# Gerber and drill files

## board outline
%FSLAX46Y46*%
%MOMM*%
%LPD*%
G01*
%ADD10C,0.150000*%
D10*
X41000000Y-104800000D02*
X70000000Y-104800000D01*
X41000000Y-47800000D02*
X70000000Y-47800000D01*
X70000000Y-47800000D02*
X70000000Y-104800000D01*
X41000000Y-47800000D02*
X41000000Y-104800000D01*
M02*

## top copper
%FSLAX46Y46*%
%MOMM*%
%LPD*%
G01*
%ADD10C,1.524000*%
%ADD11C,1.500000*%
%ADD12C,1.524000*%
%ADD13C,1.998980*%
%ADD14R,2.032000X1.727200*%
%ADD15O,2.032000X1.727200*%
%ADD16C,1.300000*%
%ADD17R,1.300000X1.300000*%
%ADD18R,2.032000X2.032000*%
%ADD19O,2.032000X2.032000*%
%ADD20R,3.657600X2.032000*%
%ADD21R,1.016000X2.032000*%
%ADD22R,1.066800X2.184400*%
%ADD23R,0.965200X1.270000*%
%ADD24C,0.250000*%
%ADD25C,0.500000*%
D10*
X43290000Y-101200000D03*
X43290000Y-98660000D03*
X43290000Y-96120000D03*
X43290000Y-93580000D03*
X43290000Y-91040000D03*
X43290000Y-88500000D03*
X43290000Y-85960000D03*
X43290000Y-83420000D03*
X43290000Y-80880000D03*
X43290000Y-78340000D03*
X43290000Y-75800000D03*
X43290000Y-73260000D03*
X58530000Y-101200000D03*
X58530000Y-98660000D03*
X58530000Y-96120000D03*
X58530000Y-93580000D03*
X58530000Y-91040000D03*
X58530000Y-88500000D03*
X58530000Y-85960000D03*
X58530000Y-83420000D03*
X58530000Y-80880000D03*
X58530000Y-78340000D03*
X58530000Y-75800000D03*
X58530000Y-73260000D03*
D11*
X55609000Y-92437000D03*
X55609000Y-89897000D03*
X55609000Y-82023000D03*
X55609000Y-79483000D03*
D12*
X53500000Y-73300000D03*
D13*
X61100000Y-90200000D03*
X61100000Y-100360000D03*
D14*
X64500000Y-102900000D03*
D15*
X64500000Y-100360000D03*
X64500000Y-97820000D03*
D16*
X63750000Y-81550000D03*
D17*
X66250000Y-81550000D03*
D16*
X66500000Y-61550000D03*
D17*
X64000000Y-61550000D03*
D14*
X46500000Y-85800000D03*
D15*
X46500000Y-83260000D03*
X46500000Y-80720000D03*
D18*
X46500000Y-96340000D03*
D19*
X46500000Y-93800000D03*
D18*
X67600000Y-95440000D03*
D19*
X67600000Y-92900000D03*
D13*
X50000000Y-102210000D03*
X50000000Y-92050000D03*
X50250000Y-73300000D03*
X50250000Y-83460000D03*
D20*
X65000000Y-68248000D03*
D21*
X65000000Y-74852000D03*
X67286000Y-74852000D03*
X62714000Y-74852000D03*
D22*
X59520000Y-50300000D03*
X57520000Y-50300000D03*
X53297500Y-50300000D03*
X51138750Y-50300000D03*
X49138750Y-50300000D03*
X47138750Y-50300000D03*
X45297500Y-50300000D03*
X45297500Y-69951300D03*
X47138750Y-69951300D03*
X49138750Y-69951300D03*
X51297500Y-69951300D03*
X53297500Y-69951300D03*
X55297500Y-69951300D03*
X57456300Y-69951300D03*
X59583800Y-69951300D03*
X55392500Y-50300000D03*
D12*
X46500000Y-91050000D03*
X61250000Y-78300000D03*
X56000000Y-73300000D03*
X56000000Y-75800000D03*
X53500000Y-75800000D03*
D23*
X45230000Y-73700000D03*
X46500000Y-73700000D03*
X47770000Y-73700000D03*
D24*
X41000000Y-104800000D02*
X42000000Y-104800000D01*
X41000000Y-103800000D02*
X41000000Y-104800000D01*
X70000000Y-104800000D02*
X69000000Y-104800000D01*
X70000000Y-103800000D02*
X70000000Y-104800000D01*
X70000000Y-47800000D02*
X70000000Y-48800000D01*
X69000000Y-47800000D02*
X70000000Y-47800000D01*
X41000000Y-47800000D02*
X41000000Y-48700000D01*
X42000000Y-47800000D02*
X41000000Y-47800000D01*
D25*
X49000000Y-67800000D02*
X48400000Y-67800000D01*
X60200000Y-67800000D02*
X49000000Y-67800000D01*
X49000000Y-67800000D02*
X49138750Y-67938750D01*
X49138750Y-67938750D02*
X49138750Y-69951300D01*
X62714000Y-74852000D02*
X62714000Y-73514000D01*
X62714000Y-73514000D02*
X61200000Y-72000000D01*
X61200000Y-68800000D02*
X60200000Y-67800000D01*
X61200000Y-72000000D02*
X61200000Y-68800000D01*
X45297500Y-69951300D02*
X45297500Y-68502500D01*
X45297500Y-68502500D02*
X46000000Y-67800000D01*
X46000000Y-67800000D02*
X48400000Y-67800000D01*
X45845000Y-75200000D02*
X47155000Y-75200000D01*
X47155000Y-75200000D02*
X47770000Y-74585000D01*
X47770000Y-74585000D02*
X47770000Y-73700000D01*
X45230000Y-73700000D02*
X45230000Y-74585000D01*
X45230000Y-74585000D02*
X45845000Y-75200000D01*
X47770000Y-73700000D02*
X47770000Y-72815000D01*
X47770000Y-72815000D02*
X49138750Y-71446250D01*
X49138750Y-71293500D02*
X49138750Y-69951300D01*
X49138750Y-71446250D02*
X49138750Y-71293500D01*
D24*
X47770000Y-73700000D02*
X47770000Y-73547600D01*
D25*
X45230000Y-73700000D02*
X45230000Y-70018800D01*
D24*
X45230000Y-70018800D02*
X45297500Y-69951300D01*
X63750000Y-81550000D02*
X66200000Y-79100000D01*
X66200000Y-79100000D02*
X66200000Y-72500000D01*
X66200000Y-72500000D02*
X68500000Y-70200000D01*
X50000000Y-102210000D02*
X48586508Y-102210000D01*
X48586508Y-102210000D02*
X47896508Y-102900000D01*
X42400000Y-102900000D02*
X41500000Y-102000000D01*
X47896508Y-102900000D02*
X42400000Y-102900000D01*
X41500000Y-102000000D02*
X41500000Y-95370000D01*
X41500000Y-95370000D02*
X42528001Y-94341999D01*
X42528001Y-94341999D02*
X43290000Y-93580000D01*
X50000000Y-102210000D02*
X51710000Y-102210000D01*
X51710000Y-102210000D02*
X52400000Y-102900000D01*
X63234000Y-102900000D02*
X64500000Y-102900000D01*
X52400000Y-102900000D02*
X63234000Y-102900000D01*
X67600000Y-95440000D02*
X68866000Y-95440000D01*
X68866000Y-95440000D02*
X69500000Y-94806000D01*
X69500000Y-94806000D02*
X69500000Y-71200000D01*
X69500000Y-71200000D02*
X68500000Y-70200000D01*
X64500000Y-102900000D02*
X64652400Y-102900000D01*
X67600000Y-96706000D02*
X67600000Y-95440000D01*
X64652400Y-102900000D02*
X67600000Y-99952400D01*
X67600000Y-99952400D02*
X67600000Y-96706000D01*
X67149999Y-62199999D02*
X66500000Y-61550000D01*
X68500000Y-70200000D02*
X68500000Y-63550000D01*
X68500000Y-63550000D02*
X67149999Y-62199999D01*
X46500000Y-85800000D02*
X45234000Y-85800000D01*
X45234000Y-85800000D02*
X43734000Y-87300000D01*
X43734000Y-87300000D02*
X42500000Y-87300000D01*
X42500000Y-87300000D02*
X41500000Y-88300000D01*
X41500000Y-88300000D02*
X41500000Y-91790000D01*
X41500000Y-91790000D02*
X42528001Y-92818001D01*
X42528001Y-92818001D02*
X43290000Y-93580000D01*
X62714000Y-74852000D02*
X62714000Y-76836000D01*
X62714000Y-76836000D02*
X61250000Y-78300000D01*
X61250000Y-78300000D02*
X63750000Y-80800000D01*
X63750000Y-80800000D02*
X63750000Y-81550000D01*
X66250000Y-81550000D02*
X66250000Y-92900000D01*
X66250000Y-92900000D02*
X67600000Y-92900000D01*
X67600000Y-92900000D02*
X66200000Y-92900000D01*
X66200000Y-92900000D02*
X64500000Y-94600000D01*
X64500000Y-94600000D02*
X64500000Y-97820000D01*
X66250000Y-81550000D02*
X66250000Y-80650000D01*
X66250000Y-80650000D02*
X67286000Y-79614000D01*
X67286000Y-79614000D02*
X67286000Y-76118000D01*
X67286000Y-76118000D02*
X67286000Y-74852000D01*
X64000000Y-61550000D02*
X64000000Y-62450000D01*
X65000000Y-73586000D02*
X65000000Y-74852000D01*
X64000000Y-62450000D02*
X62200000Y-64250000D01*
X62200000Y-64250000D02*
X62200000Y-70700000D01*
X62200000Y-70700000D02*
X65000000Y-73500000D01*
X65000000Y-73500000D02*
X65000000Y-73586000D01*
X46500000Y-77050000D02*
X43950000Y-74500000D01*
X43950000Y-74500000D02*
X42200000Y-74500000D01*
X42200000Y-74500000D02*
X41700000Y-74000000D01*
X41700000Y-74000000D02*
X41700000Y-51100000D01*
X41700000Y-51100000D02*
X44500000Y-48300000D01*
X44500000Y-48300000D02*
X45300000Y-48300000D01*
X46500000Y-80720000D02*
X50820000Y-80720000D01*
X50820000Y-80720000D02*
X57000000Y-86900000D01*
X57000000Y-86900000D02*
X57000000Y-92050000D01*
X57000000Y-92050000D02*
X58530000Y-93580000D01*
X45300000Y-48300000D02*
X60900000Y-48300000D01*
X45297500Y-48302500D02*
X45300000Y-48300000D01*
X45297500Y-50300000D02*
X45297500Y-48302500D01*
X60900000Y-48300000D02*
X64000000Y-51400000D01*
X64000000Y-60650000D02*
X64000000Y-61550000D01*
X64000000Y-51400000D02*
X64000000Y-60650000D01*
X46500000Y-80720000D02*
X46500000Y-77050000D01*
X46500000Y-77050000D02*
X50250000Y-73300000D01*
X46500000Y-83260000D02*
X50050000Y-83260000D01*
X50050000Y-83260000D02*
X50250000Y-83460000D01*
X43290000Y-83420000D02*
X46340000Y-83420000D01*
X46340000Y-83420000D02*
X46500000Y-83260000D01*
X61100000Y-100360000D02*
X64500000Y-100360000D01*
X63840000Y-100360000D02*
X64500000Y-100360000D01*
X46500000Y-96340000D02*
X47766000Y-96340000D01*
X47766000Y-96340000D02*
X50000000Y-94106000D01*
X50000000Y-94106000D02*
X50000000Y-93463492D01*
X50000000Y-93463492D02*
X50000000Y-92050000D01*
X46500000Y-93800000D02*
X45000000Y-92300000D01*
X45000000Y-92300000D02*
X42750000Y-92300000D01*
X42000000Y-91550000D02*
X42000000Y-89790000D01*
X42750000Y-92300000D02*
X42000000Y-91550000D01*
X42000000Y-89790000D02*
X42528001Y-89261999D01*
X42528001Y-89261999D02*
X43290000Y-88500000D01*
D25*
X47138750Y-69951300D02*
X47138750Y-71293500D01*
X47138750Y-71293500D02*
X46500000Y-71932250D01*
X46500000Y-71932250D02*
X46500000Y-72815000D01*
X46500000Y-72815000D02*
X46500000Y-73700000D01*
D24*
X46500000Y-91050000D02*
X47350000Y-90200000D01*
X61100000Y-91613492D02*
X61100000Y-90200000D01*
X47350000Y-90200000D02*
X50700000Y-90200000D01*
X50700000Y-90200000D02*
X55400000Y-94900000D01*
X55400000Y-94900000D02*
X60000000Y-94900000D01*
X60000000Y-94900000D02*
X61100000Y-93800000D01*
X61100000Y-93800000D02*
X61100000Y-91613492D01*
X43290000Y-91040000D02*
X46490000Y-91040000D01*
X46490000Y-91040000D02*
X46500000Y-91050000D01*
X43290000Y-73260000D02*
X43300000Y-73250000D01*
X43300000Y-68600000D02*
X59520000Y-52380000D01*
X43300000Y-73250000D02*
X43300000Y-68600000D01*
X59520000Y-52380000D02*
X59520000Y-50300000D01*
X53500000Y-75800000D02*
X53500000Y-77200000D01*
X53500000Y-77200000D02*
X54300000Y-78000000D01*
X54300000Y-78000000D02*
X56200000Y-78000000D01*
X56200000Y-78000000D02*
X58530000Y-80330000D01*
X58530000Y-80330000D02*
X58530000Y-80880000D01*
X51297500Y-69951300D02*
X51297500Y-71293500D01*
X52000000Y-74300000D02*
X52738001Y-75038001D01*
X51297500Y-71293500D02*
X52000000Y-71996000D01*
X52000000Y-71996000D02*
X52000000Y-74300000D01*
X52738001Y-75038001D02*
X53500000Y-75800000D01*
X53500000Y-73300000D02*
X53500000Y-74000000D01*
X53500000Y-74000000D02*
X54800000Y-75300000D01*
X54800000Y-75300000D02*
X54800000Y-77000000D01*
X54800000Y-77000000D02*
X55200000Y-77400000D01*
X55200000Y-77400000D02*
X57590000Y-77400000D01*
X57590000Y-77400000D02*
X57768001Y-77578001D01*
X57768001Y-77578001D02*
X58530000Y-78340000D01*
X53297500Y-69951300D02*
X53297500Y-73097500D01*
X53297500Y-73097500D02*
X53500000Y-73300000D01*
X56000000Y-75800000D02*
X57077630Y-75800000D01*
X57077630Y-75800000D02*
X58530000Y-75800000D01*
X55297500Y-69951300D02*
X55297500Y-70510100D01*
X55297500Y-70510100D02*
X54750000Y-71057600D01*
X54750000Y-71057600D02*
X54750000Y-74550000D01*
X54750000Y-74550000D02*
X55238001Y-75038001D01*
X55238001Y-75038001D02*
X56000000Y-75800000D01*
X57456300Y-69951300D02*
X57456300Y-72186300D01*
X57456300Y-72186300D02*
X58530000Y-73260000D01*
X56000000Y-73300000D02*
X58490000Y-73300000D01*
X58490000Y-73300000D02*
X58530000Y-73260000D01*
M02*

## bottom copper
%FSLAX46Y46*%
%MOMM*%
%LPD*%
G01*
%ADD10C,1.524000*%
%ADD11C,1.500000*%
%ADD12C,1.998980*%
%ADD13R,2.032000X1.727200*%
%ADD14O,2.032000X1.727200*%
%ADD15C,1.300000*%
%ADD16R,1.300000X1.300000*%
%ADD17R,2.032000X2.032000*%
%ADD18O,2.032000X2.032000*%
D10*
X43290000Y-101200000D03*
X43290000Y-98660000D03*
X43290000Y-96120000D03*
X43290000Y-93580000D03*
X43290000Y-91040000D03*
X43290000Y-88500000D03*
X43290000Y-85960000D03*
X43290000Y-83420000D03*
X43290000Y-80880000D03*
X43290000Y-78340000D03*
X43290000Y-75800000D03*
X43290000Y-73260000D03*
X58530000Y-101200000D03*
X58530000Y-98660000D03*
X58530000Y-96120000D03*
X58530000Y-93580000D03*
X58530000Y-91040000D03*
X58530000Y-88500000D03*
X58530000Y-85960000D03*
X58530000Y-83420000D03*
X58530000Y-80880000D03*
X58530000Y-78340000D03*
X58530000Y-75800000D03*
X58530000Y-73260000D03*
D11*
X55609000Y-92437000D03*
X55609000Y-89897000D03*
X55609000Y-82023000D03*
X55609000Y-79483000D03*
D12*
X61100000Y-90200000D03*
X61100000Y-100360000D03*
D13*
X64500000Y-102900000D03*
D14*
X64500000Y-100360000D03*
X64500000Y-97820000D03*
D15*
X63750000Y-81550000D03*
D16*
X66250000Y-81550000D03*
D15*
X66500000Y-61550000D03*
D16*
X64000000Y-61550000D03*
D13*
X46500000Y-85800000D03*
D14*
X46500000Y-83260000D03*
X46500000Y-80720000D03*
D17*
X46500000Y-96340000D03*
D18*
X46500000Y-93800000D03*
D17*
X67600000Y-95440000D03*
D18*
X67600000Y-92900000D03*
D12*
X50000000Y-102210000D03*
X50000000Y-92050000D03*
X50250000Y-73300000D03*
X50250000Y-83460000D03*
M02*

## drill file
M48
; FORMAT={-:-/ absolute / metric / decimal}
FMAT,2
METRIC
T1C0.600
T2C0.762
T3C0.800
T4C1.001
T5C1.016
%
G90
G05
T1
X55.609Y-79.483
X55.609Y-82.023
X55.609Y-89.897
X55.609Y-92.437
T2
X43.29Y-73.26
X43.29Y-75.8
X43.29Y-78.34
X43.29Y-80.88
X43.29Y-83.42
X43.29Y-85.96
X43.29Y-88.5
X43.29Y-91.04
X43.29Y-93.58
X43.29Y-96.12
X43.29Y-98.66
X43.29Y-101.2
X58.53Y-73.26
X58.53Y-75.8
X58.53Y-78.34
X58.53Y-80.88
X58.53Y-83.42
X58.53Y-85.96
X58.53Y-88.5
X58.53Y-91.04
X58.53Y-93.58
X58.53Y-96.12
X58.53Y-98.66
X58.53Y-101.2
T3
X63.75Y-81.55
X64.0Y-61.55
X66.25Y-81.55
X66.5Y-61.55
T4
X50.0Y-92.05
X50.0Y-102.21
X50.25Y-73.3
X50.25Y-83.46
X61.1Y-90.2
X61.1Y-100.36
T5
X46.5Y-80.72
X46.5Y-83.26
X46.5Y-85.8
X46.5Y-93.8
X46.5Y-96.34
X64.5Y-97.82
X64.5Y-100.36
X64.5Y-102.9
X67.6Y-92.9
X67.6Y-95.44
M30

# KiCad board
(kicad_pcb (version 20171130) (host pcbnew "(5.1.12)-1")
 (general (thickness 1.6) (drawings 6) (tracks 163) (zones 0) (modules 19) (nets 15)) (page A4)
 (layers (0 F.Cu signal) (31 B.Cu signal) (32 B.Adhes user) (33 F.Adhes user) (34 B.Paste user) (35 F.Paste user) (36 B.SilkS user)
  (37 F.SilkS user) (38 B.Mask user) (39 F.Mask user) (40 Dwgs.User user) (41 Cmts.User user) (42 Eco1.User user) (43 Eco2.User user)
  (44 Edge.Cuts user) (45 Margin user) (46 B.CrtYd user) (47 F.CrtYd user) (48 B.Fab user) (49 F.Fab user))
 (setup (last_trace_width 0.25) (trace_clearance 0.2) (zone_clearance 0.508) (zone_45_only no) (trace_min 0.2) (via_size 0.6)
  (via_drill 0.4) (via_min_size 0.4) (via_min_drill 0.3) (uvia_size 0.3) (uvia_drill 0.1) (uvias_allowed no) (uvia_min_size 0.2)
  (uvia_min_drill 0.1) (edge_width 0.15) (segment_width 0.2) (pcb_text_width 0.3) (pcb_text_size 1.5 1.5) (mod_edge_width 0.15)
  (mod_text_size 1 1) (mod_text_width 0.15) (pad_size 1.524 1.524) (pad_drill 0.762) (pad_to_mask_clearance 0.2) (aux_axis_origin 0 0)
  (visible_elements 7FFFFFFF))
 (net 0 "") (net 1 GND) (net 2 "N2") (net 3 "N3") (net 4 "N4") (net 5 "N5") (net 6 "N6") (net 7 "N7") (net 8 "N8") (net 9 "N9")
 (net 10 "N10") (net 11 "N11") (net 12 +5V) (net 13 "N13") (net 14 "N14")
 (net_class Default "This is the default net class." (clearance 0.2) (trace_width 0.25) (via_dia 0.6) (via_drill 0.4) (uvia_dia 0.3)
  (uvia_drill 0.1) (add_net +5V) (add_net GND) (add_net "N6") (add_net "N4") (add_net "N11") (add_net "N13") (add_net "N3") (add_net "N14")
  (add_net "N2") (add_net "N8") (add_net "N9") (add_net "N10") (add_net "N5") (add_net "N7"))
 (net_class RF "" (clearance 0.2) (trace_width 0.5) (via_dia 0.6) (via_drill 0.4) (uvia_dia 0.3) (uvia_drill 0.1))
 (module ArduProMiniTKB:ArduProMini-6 (layer B.Cu) (at 40.75 107.55)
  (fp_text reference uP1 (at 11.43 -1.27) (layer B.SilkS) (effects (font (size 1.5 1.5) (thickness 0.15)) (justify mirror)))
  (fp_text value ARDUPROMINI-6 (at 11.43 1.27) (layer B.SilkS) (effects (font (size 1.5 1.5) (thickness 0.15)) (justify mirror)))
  (pad 7 thru_hole circle (at 2.54 -6.35) (size 1.524 1.524) (drill 0.762) (layers *.Cu *.Mask B.SilkS))
  (pad 8 thru_hole circle (at 2.54 -8.89) (size 1.524 1.524) (drill 0.762) (layers *.Cu *.Mask B.SilkS))
  (pad 9 thru_hole circle (at 2.54 -11.43) (size 1.524 1.524) (drill 0.762) (layers *.Cu *.Mask B.SilkS))
  (pad 10 thru_hole circle (at 2.54 -13.97) (size 1.524 1.524) (drill 0.762) (layers *.Cu *.Mask B.SilkS) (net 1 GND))
  (pad 11 thru_hole circle (at 2.54 -16.51) (size 1.524 1.524) (drill 0.762) (layers *.Cu *.Mask B.SilkS) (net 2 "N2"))
  (pad 12 thru_hole circle (at 2.54 -19.05) (size 1.524 1.524) (drill 0.762) (layers *.Cu *.Mask B.SilkS) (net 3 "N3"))
  (pad 13 thru_hole circle (at 2.54 -21.59) (size 1.524 1.524) (drill 0.762) (layers *.Cu *.Mask B.SilkS))
  (pad 14 thru_hole circle (at 2.54 -24.13) (size 1.524 1.524) (drill 0.762) (layers *.Cu *.Mask B.SilkS) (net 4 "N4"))
  (pad 15 thru_hole circle (at 2.54 -26.67) (size 1.524 1.524) (drill 0.762) (layers *.Cu *.Mask B.SilkS))
  (pad 16 thru_hole circle (at 2.54 -29.21) (size 1.524 1.524) (drill 0.762) (layers *.Cu *.Mask B.SilkS))
  (pad 17 thru_hole circle (at 2.54 -31.75) (size 1.524 1.524) (drill 0.762) (layers *.Cu *.Mask B.SilkS))
  (pad 18 thru_hole circle (at 2.54 -34.29) (size 1.524 1.524) (drill 0.762) (layers *.Cu *.Mask B.SilkS) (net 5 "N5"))
  (pad 19 thru_hole circle (at 17.78 -6.35) (size 1.524 1.524) (drill 0.762) (layers *.Cu *.Mask B.SilkS))
  (pad 20 thru_hole circle (at 17.78 -8.89) (size 1.524 1.524) (drill 0.762) (layers *.Cu *.Mask B.SilkS))
  (pad 21 thru_hole circle (at 17.78 -11.43) (size 1.524 1.524) (drill 0.762) (layers *.Cu *.Mask B.SilkS))
  (pad 22 thru_hole circle (at 17.78 -13.97) (size 1.524 1.524) (drill 0.762) (layers *.Cu *.Mask B.SilkS) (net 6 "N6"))
  (pad 23 thru_hole circle (at 17.78 -16.51) (size 1.524 1.524) (drill 0.762) (layers *.Cu *.Mask B.SilkS))
  (pad 24 thru_hole circle (at 17.78 -19.05) (size 1.524 1.524) (drill 0.762) (layers *.Cu *.Mask B.SilkS))
  (pad 25 thru_hole circle (at 17.78 -21.59) (size 1.524 1.524) (drill 0.762) (layers *.Cu *.Mask B.SilkS))
  (pad 26 thru_hole circle (at 17.78 -24.13) (size 1.524 1.524) (drill 0.762) (layers *.Cu *.Mask B.SilkS))
  (pad 27 thru_hole circle (at 17.78 -26.67) (size 1.524 1.524) (drill 0.762) (layers *.Cu *.Mask B.SilkS) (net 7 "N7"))
  (pad 28 thru_hole circle (at 17.78 -29.21) (size 1.524 1.524) (drill 0.762) (layers *.Cu *.Mask B.SilkS) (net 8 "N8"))
  (pad 29 thru_hole circle (at 17.78 -31.75) (size 1.524 1.524) (drill 0.762) (layers *.Cu *.Mask B.SilkS) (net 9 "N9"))
  (pad 30 thru_hole circle (at 17.78 -34.29) (size 1.524 1.524) (drill 0.762) (layers *.Cu *.Mask B.SilkS) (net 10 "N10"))
  (pad 31 thru_hole circle (at 14.859 -15.113) (size 1.5 1.5) (drill 0.6) (layers *.Cu *.Mask B.SilkS))
  (pad 32 thru_hole circle (at 14.859 -17.653) (size 1.5 1.5) (drill 0.6) (layers *.Cu *.Mask B.SilkS))
  (pad 34 thru_hole circle (at 14.859 -25.527) (size 1.5 1.5) (drill 0.6) (layers *.Cu *.Mask B.SilkS))
  (pad 35 thru_hole circle (at 14.859 -28.067) (size 1.5 1.5) (drill 0.6) (layers *.Cu *.Mask B.SilkS)))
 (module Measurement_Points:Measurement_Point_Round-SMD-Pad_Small (layer F.Cu) (at 53.5 73.3)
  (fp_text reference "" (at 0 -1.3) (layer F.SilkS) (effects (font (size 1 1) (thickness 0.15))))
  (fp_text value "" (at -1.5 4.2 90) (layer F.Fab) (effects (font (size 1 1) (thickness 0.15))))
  (pad 1 smd circle (at 0 0) (size 1.524 1.524) (layers F.Cu F.Paste F.Mask) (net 8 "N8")))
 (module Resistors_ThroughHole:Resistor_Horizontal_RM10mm (layer F.Cu) (at 61.1 90.2 270)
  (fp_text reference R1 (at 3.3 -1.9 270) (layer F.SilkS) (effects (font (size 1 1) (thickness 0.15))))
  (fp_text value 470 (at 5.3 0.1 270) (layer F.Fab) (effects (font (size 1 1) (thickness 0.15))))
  (pad 1 thru_hole circle (at 0 0 270) (size 1.99898 1.99898) (drill 1.00076) (layers *.Cu *.SilkS *.Mask) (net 2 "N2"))
  (pad 2 thru_hole circle (at 10.16 0 270) (size 1.99898 1.99898) (drill 1.00076) (layers *.Cu *.SilkS *.Mask) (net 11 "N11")))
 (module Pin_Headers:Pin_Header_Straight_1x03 (layer F.Cu) (at 64.5 102.9 180)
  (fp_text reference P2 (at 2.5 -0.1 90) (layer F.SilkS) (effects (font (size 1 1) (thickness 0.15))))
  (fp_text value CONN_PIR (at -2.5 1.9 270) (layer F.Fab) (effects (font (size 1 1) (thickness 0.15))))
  (pad 1 thru_hole rect (at 0 0 180) (size 2.032 1.7272) (drill 1.016) (layers *.Cu *.Mask F.SilkS) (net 1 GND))
  (pad 2 thru_hole oval (at 0 2.54 180) (size 2.032 1.7272) (drill 1.016) (layers *.Cu *.Mask F.SilkS) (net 11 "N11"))
  (pad 3 thru_hole oval (at 0 5.08 180) (size 2.032 1.7272) (drill 1.016) (layers *.Cu *.Mask F.SilkS) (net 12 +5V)))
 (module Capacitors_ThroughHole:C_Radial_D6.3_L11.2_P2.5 (layer F.Cu) (at 66.25 81.55 180)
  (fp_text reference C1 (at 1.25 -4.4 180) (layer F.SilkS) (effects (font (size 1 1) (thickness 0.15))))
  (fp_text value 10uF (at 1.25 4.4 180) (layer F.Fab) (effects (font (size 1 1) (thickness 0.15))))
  (pad 2 thru_hole circle (at 2.5 0 180) (size 1.3 1.3) (drill 0.8) (layers *.Cu *.Mask F.SilkS) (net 1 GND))
  (pad 1 thru_hole rect (at 0 0 180) (size 1.3 1.3) (drill 0.8) (layers *.Cu *.Mask F.SilkS) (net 12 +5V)))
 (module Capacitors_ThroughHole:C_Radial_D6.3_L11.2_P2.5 (layer F.Cu) (at 64 61.55)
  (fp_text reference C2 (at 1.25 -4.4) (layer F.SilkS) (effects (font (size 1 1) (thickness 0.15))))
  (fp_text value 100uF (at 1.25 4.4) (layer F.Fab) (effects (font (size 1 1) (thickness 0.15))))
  (pad 2 thru_hole circle (at 2.5 0) (size 1.3 1.3) (drill 0.8) (layers *.Cu *.Mask F.SilkS) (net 1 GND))
  (pad 1 thru_hole rect (at 0 0) (size 1.3 1.3) (drill 0.8) (layers *.Cu *.Mask F.SilkS) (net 6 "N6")))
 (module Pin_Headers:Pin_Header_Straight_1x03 (layer F.Cu) (at 46.5 85.8 180)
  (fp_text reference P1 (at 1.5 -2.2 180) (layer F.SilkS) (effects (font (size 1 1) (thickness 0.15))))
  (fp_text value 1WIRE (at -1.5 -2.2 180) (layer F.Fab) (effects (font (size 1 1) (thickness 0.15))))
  (pad 1 thru_hole rect (at 0 0 180) (size 2.032 1.7272) (drill 1.016) (layers *.Cu *.Mask F.SilkS) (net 1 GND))
  (pad 2 thru_hole oval (at 0 2.54 180) (size 2.032 1.7272) (drill 1.016) (layers *.Cu *.Mask F.SilkS) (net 4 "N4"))
  (pad 3 thru_hole oval (at 0 5.08 180) (size 2.032 1.7272) (drill 1.016) (layers *.Cu *.Mask F.SilkS) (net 6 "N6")))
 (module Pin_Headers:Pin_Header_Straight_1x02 (layer F.Cu) (at 46.5 96.34 180)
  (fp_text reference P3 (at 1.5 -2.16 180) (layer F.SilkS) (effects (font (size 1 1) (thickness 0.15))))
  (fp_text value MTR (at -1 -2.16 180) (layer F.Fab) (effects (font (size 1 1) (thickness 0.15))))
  (pad 1 thru_hole rect (at 0 0 180) (size 2.032 2.032) (drill 1.016) (layers *.Cu *.Mask F.SilkS) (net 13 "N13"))
  (pad 2 thru_hole oval (at 0 2.54 180) (size 2.032 2.032) (drill 1.016) (layers *.Cu *.Mask F.SilkS) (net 3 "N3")))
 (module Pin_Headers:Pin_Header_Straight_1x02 (layer F.Cu) (at 67.6 95.44 180)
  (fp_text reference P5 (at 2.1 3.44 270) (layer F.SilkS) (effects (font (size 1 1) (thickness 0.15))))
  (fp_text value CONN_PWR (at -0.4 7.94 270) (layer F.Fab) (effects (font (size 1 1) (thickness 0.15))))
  (pad 1 thru_hole rect (at 0 0 180) (size 2.032 2.032) (drill 1.016) (layers *.Cu *.Mask F.SilkS) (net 1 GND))
  (pad 2 thru_hole oval (at 0 2.54 180) (size 2.032 2.032) (drill 1.016) (layers *.Cu *.Mask F.SilkS) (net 12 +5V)))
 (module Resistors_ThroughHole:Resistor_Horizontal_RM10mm (layer F.Cu) (at 50 102.21 90)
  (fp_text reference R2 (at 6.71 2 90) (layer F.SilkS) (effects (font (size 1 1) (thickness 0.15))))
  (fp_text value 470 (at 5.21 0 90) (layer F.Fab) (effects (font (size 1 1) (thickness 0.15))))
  (pad 1 thru_hole circle (at 0 0 90) (size 1.99898 1.99898) (drill 1.00076) (layers *.Cu *.SilkS *.Mask) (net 1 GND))
  (pad 2 thru_hole circle (at 10.16 0 90) (size 1.99898 1.99898) (drill 1.00076) (layers *.Cu *.SilkS *.Mask) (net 13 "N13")))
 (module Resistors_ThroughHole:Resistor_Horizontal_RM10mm (layer F.Cu) (at 50.25 73.3 270)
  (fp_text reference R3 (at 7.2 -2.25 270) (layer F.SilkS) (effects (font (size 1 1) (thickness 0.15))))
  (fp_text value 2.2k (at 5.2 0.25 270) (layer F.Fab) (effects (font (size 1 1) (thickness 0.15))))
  (pad 1 thru_hole circle (at 0 0 270) (size 1.99898 1.99898) (drill 1.00076) (layers *.Cu *.SilkS *.Mask) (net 6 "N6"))
  (pad 2 thru_hole circle (at 10.16 0 270) (size 1.99898 1.99898) (drill 1.00076) (layers *.Cu *.SilkS *.Mask) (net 4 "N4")))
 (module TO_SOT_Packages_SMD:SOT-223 (layer F.Cu) (at 65 71.55)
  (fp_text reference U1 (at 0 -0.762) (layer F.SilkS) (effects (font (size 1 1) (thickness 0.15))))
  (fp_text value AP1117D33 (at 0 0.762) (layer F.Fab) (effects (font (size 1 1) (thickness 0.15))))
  (pad 4 smd rect (at 0 -3.302) (size 3.6576 2.032) (layers F.Cu F.Paste F.Mask))
  (pad 2 smd rect (at 0 3.302) (size 1.016 2.032) (layers F.Cu F.Paste F.Mask) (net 6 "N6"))
  (pad 3 smd rect (at 2.286 3.302) (size 1.016 2.032) (layers F.Cu F.Paste F.Mask) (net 12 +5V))
  (pad 1 smd rect (at -2.286 3.302) (size 1.016 2.032) (layers F.Cu F.Paste F.Mask) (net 1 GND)))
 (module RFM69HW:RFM (layer F.Cu) (at 44.25 50.3 270) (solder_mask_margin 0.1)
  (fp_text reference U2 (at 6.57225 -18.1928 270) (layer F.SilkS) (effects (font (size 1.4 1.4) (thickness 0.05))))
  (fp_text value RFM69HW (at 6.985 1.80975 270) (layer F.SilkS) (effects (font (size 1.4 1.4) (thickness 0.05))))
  (pad RESE smd rect (at 0 -15.27 270) (size 2.1844 1.0668) (layers F.Cu F.Paste F.Mask) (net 5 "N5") (solder_mask_margin 0.2))
  (pad DIO0 smd rect (at 0 -13.27 270) (size 2.1844 1.0668) (layers F.Cu F.Paste F.Mask) (solder_mask_margin 0.2))
  (pad DIO2 smd rect (at 0 -9.0475 270) (size 2.1844 1.0668) (layers F.Cu F.Paste F.Mask) (solder_mask_margin 0.2))
  (pad DIO3 smd rect (at 0 -6.88875 270) (size 2.1844 1.0668) (layers F.Cu F.Paste F.Mask) (solder_mask_margin 0.2))
  (pad DIO4 smd rect (at 0 -4.88875 270) (size 2.1844 1.0668) (layers F.Cu F.Paste F.Mask) (solder_mask_margin 0.2))
  (pad DIO5 smd rect (at 0 -2.88875 270) (size 2.1844 1.0668) (layers F.Cu F.Paste F.Mask) (solder_mask_margin 0.2))
  (pad VCC smd rect (at 0 -1.0475 270) (size 2.1844 1.0668) (layers F.Cu F.Paste F.Mask) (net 6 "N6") (solder_mask_margin 0.2))
  (pad GNDB smd rect (at 19.6513 -1.0475 270) (size 2.1844 1.0668) (layers F.Cu F.Paste F.Mask) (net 1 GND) (solder_mask_margin 0.2))
  (pad ANT smd rect (at 19.6513 -2.88875 270) (size 2.1844 1.0668) (layers F.Cu F.Paste F.Mask) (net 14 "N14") (solder_mask_margin 0.2))
  (pad GNDA smd rect (at 19.6513 -4.88875 270) (size 2.1844 1.0668) (layers F.Cu F.Paste F.Mask) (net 1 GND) (solder_mask_margin 0.2))
  (pad SCK smd rect (at 19.6513 -7.0475 270) (size 2.1844 1.0668) (layers F.Cu F.Paste F.Mask) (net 7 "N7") (solder_mask_margin 0.2))
  (pad MISO smd rect (at 19.6513 -9.0475 270) (size 2.1844 1.0668) (layers F.Cu F.Paste F.Mask) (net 8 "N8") (solder_mask_margin 0.2))
  (pad MOSI smd rect (at 19.6513 -11.0475 270) (size 2.1844 1.0668) (layers F.Cu F.Paste F.Mask) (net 9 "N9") (solder_mask_margin 0.2))
  (pad NSS smd rect (at 19.6513 -13.2063 270) (size 2.1844 1.0668) (layers F.Cu F.Paste F.Mask) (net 10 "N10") (solder_mask_margin 0.2))
  (pad NC smd rect (at 19.6513 -15.3338 270) (size 2.1844 1.0668) (layers F.Cu F.Paste F.Mask) (solder_mask_margin 0.2))
  (pad DIO1 smd rect (at 0 -11.1425 270) (size 2.1844 1.0668) (layers F.Cu F.Paste F.Mask) (solder_mask_margin 0.2)))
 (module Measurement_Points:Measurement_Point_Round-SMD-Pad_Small (layer F.Cu) (at 46.5 91.05)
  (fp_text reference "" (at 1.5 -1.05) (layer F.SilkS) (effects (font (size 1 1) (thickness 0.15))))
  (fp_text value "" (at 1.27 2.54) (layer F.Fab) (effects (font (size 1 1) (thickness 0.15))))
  (pad 1 smd circle (at 0 0) (size 1.524 1.524) (layers F.Cu F.Paste F.Mask) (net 2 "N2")))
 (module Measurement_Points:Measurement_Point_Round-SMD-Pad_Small (layer F.Cu) (at 61.25 78.3)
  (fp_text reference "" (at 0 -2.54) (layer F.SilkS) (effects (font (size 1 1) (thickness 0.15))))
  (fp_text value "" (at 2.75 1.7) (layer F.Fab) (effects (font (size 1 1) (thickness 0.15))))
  (pad 1 smd circle (at 0 0) (size 1.524 1.524) (layers F.Cu F.Paste F.Mask) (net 1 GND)))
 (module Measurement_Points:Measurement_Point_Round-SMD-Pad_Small (layer F.Cu) (at 56 73.3)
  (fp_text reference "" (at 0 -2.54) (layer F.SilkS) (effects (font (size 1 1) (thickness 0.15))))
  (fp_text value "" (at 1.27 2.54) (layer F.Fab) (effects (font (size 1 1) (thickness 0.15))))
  (pad 1 smd circle (at 0 0) (size 1.524 1.524) (layers F.Cu F.Paste F.Mask) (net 10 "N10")))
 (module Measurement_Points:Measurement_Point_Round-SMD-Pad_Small (layer F.Cu) (at 56 75.8)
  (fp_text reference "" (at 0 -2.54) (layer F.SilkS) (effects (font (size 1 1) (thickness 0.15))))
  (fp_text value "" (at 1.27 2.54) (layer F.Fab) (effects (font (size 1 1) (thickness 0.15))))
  (pad 1 smd circle (at 0 0) (size 1.524 1.524) (layers F.Cu F.Paste F.Mask) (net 9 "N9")))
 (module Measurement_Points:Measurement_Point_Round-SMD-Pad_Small (layer F.Cu) (at 53.5 75.8)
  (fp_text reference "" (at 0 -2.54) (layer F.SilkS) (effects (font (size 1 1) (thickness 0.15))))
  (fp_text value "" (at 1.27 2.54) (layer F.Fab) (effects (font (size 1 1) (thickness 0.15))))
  (pad 1 smd circle (at 0 0) (size 1.524 1.524) (layers F.Cu F.Paste F.Mask) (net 7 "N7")))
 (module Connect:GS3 (layer F.Cu) (at 46.5 73.7 90)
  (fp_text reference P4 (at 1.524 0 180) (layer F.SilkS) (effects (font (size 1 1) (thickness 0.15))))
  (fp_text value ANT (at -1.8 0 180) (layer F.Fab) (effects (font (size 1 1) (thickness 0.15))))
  (pad 1 smd rect (at 0 -1.27 90) (size 1.27 0.9652) (layers F.Cu F.Paste F.Mask) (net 1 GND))
  (pad 2 smd rect (at 0 0 90) (size 1.27 0.9652) (layers F.Cu F.Paste F.Mask) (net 14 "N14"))
  (pad 3 smd rect (at 0 1.27 90) (size 1.27 0.9652) (layers F.Cu F.Paste F.Mask) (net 1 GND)))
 (gr_line (start 41 104.8) (end 70 104.8) (angle 90) (layer Edge.Cuts) (width 0.15))
 (gr_line (start 41 47.8) (end 70 47.8) (angle 90) (layer Edge.Cuts) (width 0.15))
 (gr_line (start 70 47.8) (end 70 104.8) (angle 90) (layer Edge.Cuts) (width 0.15))
 (gr_line (start 41 47.8) (end 41 104.8) (angle 90) (layer Edge.Cuts) (width 0.15))
 (segment (start 41 104.8) (end 42 104.8) (width 0.25) (layer F.Cu) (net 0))
 (segment (start 41 103.8) (end 41 104.8) (width 0.25) (layer F.Cu) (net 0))
 (segment (start 70 104.8) (end 69 104.8) (width 0.25) (layer F.Cu) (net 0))
 (segment (start 70 103.8) (end 70 104.8) (width 0.25) (layer F.Cu) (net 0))
 (segment (start 70 47.8) (end 70 48.8) (width 0.25) (layer F.Cu) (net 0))
 (segment (start 69 47.8) (end 70 47.8) (width 0.25) (layer F.Cu) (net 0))
 (segment (start 41 47.8) (end 41 48.7) (width 0.25) (layer F.Cu) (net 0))
 (segment (start 42 47.8) (end 41 47.8) (width 0.25) (layer F.Cu) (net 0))
 (segment (start 49 67.8) (end 48.4 67.8) (width 0.5) (layer F.Cu) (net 1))
 (segment (start 60.2 67.8) (end 49 67.8) (width 0.5) (layer F.Cu) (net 1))
 (segment (start 49 67.8) (end 49.13875 67.93875) (width 0.5) (layer F.Cu) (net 1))
 (segment (start 49.13875 67.93875) (end 49.13875 69.9513) (width 0.5) (layer F.Cu) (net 1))
 (segment (start 62.714 74.852) (end 62.714 73.514) (width 0.5) (layer F.Cu) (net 1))
 (segment (start 62.714 73.514) (end 61.2 72) (width 0.5) (layer F.Cu) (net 1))
 (segment (start 61.2 68.8) (end 60.2 67.8) (width 0.5) (layer F.Cu) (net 1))
 (segment (start 61.2 72) (end 61.2 68.8) (width 0.5) (layer F.Cu) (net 1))
 (segment (start 45.2975 69.9513) (end 45.2975 68.5025) (width 0.5) (layer F.Cu) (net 1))
 (segment (start 45.2975 68.5025) (end 46 67.8) (width 0.5) (layer F.Cu) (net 1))
 (segment (start 46 67.8) (end 48.4 67.8) (width 0.5) (layer F.Cu) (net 1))
 (segment (start 45.845 75.2) (end 47.155 75.2) (width 0.5) (layer F.Cu) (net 1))
 (segment (start 47.155 75.2) (end 47.77 74.585) (width 0.5) (layer F.Cu) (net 1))
 (segment (start 47.77 74.585) (end 47.77 73.7) (width 0.5) (layer F.Cu) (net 1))
 (segment (start 45.23 73.7) (end 45.23 74.585) (width 0.5) (layer F.Cu) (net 1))
 (segment (start 45.23 74.585) (end 45.845 75.2) (width 0.5) (layer F.Cu) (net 1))
 (segment (start 47.77 73.7) (end 47.77 72.815) (width 0.5) (layer F.Cu) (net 1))
 (segment (start 47.77 72.815) (end 49.13875 71.44625) (width 0.5) (layer F.Cu) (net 1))
 (segment (start 49.13875 71.2935) (end 49.13875 69.9513) (width 0.5) (layer F.Cu) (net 1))
 (segment (start 49.13875 71.44625) (end 49.13875 71.2935) (width 0.5) (layer F.Cu) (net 1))
 (segment (start 47.77 73.7) (end 47.77 73.5476) (width 0.25) (layer F.Cu) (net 1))
 (segment (start 45.23 73.7) (end 45.23 70.0188) (width 0.5) (layer F.Cu) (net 1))
 (segment (start 45.23 70.0188) (end 45.2975 69.9513) (width 0.25) (layer F.Cu) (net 1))
 (segment (start 63.75 81.55) (end 66.2 79.1) (width 0.25) (layer F.Cu) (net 1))
 (segment (start 66.2 79.1) (end 66.2 72.5) (width 0.25) (layer F.Cu) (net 1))
 (segment (start 66.2 72.5) (end 68.5 70.2) (width 0.25) (layer F.Cu) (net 1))
 (segment (start 50 102.21) (end 48.586508 102.21) (width 0.25) (layer F.Cu) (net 1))
 (segment (start 48.586508 102.21) (end 47.896508 102.9) (width 0.25) (layer F.Cu) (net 1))
 (segment (start 42.4 102.9) (end 41.5 102) (width 0.25) (layer F.Cu) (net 1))
 (segment (start 47.896508 102.9) (end 42.4 102.9) (width 0.25) (layer F.Cu) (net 1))
 (segment (start 41.5 102) (end 41.5 95.37) (width 0.25) (layer F.Cu) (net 1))
 (segment (start 41.5 95.37) (end 42.528001 94.341999) (width 0.25) (layer F.Cu) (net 1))
 (segment (start 42.528001 94.341999) (end 43.29 93.58) (width 0.25) (layer F.Cu) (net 1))
 (segment (start 50 102.21) (end 51.71 102.21) (width 0.25) (layer F.Cu) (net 1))
 (segment (start 51.71 102.21) (end 52.4 102.9) (width 0.25) (layer F.Cu) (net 1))
 (segment (start 63.234 102.9) (end 64.5 102.9) (width 0.25) (layer F.Cu) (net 1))
 (segment (start 52.4 102.9) (end 63.234 102.9) (width 0.25) (layer F.Cu) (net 1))
 (segment (start 67.6 95.44) (end 68.866 95.44) (width 0.25) (layer F.Cu) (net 1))
 (segment (start 68.866 95.44) (end 69.5 94.806) (width 0.25) (layer F.Cu) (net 1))
 (segment (start 69.5 94.806) (end 69.5 71.2) (width 0.25) (layer F.Cu) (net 1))
 (segment (start 69.5 71.2) (end 68.5 70.2) (width 0.25) (layer F.Cu) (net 1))
 (segment (start 64.5 102.9) (end 64.6524 102.9) (width 0.25) (layer F.Cu) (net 1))
 (segment (start 67.6 96.706) (end 67.6 95.44) (width 0.25) (layer F.Cu) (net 1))
 (segment (start 64.6524 102.9) (end 67.6 99.9524) (width 0.25) (layer F.Cu) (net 1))
 (segment (start 67.6 99.9524) (end 67.6 96.706) (width 0.25) (layer F.Cu) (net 1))
 (segment (start 67.149999 62.199999) (end 66.5 61.55) (width 0.25) (layer F.Cu) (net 1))
 (segment (start 68.5 70.2) (end 68.5 63.55) (width 0.25) (layer F.Cu) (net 1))
 (segment (start 68.5 63.55) (end 67.149999 62.199999) (width 0.25) (layer F.Cu) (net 1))
 (segment (start 46.5 85.8) (end 45.234 85.8) (width 0.25) (layer F.Cu) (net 1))
 (segment (start 45.234 85.8) (end 43.734 87.3) (width 0.25) (layer F.Cu) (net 1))
 (segment (start 43.734 87.3) (end 42.5 87.3) (width 0.25) (layer F.Cu) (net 1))
 (segment (start 42.5 87.3) (end 41.5 88.3) (width 0.25) (layer F.Cu) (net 1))
 (segment (start 41.5 88.3) (end 41.5 91.79) (width 0.25) (layer F.Cu) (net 1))
 (segment (start 41.5 91.79) (end 42.528001 92.818001) (width 0.25) (layer F.Cu) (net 1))
 (segment (start 42.528001 92.818001) (end 43.29 93.58) (width 0.25) (layer F.Cu) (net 1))
 (segment (start 62.714 74.852) (end 62.714 76.836) (width 0.25) (layer F.Cu) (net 1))
 (segment (start 62.714 76.836) (end 61.25 78.3) (width 0.25) (layer F.Cu) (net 1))
 (segment (start 61.25 78.3) (end 63.75 80.8) (width 0.25) (layer F.Cu) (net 1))
 (segment (start 63.75 80.8) (end 63.75 81.55) (width 0.25) (layer F.Cu) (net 1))
 (segment (start 66.25 81.55) (end 66.25 92.9) (width 0.25) (layer F.Cu) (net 12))
 (segment (start 66.25 92.9) (end 67.6 92.9) (width 0.25) (layer F.Cu) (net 12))
 (segment (start 67.6 92.9) (end 66.2 92.9) (width 0.25) (layer F.Cu) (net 12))
 (segment (start 66.2 92.9) (end 64.5 94.6) (width 0.25) (layer F.Cu) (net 12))
 (segment (start 64.5 94.6) (end 64.5 97.82) (width 0.25) (layer F.Cu) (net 12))
 (segment (start 66.25 81.55) (end 66.25 80.65) (width 0.25) (layer F.Cu) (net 12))
 (segment (start 66.25 80.65) (end 67.286 79.614) (width 0.25) (layer F.Cu) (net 12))
 (segment (start 67.286 79.614) (end 67.286 76.118) (width 0.25) (layer F.Cu) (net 12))
 (segment (start 67.286 76.118) (end 67.286 74.852) (width 0.25) (layer F.Cu) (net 12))
 (segment (start 64 61.55) (end 64 62.45) (width 0.25) (layer F.Cu) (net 6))
 (segment (start 65 73.586) (end 65 74.852) (width 0.25) (layer F.Cu) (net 6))
 (segment (start 64 62.45) (end 62.2 64.25) (width 0.25) (layer F.Cu) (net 6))
 (segment (start 62.2 64.25) (end 62.2 70.7) (width 0.25) (layer F.Cu) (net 6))
 (segment (start 62.2 70.7) (end 65 73.5) (width 0.25) (layer F.Cu) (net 6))
 (segment (start 65 73.5) (end 65 73.586) (width 0.25) (layer F.Cu) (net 6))
 (segment (start 46.5 77.05) (end 43.95 74.5) (width 0.25) (layer F.Cu) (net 6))
 (segment (start 43.95 74.5) (end 42.2 74.5) (width 0.25) (layer F.Cu) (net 6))
 (segment (start 42.2 74.5) (end 41.7 74) (width 0.25) (layer F.Cu) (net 6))
 (segment (start 41.7 74) (end 41.7 51.1) (width 0.25) (layer F.Cu) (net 6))
 (segment (start 41.7 51.1) (end 44.5 48.3) (width 0.25) (layer F.Cu) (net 6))
 (segment (start 44.5 48.3) (end 45.3 48.3) (width 0.25) (layer F.Cu) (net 6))
 (segment (start 46.5 80.72) (end 50.82 80.72) (width 0.25) (layer F.Cu) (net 6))
 (segment (start 50.82 80.72) (end 57 86.9) (width 0.25) (layer F.Cu) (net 6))
 (segment (start 57 86.9) (end 57 92.05) (width 0.25) (layer F.Cu) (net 6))
 (segment (start 57 92.05) (end 58.53 93.58) (width 0.25) (layer F.Cu) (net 6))
 (segment (start 45.3 48.3) (end 60.9 48.3) (width 0.25) (layer F.Cu) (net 6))
 (segment (start 45.2975 48.3025) (end 45.3 48.3) (width 0.25) (layer F.Cu) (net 6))
 (segment (start 45.2975 50.3) (end 45.2975 48.3025) (width 0.25) (layer F.Cu) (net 6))
 (segment (start 60.9 48.3) (end 64 51.4) (width 0.25) (layer F.Cu) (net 6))
 (segment (start 64 60.65) (end 64 61.55) (width 0.25) (layer F.Cu) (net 6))
 (segment (start 64 51.4) (end 64 60.65) (width 0.25) (layer F.Cu) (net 6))
 (segment (start 46.5 80.72) (end 46.5 77.05) (width 0.25) (layer F.Cu) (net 6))
 (segment (start 46.5 77.05) (end 50.25 73.3) (width 0.25) (layer F.Cu) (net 6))
 (segment (start 46.5 83.26) (end 50.05 83.26) (width 0.25) (layer F.Cu) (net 4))
 (segment (start 50.05 83.26) (end 50.25 83.46) (width 0.25) (layer F.Cu) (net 4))
 (segment (start 43.29 83.42) (end 46.34 83.42) (width 0.25) (layer F.Cu) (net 4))
 (segment (start 46.34 83.42) (end 46.5 83.26) (width 0.25) (layer F.Cu) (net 4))
 (segment (start 61.1 100.36) (end 64.5 100.36) (width 0.25) (layer F.Cu) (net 11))
 (segment (start 63.84 100.36) (end 64.5 100.36) (width 0.25) (layer F.Cu) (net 11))
 (segment (start 46.5 96.34) (end 47.766 96.34) (width 0.25) (layer F.Cu) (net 13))
 (segment (start 47.766 96.34) (end 50 94.106) (width 0.25) (layer F.Cu) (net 13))
 (segment (start 50 94.106) (end 50 93.463492) (width 0.25) (layer F.Cu) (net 13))
 (segment (start 50 93.463492) (end 50 92.05) (width 0.25) (layer F.Cu) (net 13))
 (segment (start 46.5 93.8) (end 45 92.3) (width 0.25) (layer F.Cu) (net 3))
 (segment (start 45 92.3) (end 42.75 92.3) (width 0.25) (layer F.Cu) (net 3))
 (segment (start 42 91.55) (end 42 89.79) (width 0.25) (layer F.Cu) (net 3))
 (segment (start 42.75 92.3) (end 42 91.55) (width 0.25) (layer F.Cu) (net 3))
 (segment (start 42 89.79) (end 42.528001 89.261999) (width 0.25) (layer F.Cu) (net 3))
 (segment (start 42.528001 89.261999) (end 43.29 88.5) (width 0.25) (layer F.Cu) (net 3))
 (segment (start 47.13875 69.9513) (end 47.13875 71.2935) (width 0.5) (layer F.Cu) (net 14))
 (segment (start 47.13875 71.2935) (end 46.5 71.93225) (width 0.5) (layer F.Cu) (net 14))
 (segment (start 46.5 71.93225) (end 46.5 72.815) (width 0.5) (layer F.Cu) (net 14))
 (segment (start 46.5 72.815) (end 46.5 73.7) (width 0.5) (layer F.Cu) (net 14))
 (segment (start 46.5 91.05) (end 47.35 90.2) (width 0.25) (layer F.Cu) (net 2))
 (segment (start 61.1 91.613492) (end 61.1 90.2) (width 0.25) (layer F.Cu) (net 2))
 (segment (start 47.35 90.2) (end 50.7 90.2) (width 0.25) (layer F.Cu) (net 2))
 (segment (start 50.7 90.2) (end 55.4 94.9) (width 0.25) (layer F.Cu) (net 2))
 (segment (start 55.4 94.9) (end 60 94.9) (width 0.25) (layer F.Cu) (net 2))
 (segment (start 60 94.9) (end 61.1 93.8) (width 0.25) (layer F.Cu) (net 2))
 (segment (start 61.1 93.8) (end 61.1 91.613492) (width 0.25) (layer F.Cu) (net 2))
 (segment (start 43.29 91.04) (end 46.49 91.04) (width 0.25) (layer F.Cu) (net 2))
 (segment (start 46.49 91.04) (end 46.5 91.05) (width 0.25) (layer F.Cu) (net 2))
 (segment (start 43.29 73.26) (end 43.3 73.25) (width 0.25) (layer F.Cu) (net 5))
 (segment (start 43.3 68.6) (end 59.52 52.38) (width 0.25) (layer F.Cu) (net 5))
 (segment (start 43.3 73.25) (end 43.3 68.6) (width 0.25) (layer F.Cu) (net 5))
 (segment (start 59.52 52.38) (end 59.52 50.3) (width 0.25) (layer F.Cu) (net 5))
 (segment (start 53.5 75.8) (end 53.5 77.2) (width 0.25) (layer F.Cu) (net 7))
 (segment (start 53.5 77.2) (end 54.3 78) (width 0.25) (layer F.Cu) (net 7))
 (segment (start 54.3 78) (end 56.2 78) (width 0.25) (layer F.Cu) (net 7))
 (segment (start 56.2 78) (end 58.53 80.33) (width 0.25) (layer F.Cu) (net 7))
 (segment (start 58.53 80.33) (end 58.53 80.88) (width 0.25) (layer F.Cu) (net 7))
 (segment (start 51.2975 69.9513) (end 51.2975 71.2935) (width 0.25) (layer F.Cu) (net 7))
 (segment (start 52 74.3) (end 52.738001 75.038001) (width 0.25) (layer F.Cu) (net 7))
 (segment (start 51.2975 71.2935) (end 52 71.996) (width 0.25) (layer F.Cu) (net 7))
 (segment (start 52 71.996) (end 52 74.3) (width 0.25) (layer F.Cu) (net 7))
 (segment (start 52.738001 75.038001) (end 53.5 75.8) (width 0.25) (layer F.Cu) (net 7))
 (segment (start 53.5 73.3) (end 53.5 74) (width 0.25) (layer F.Cu) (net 8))
 (segment (start 53.5 74) (end 54.8 75.3) (width 0.25) (layer F.Cu) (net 8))
 (segment (start 54.8 75.3) (end 54.8 77) (width 0.25) (layer F.Cu) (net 8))
 (segment (start 54.8 77) (end 55.2 77.4) (width 0.25) (layer F.Cu) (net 8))
 (segment (start 55.2 77.4) (end 57.59 77.4) (width 0.25) (layer F.Cu) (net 8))
 (segment (start 57.59 77.4) (end 57.768001 77.578001) (width 0.25) (layer F.Cu) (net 8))
 (segment (start 57.768001 77.578001) (end 58.53 78.34) (width 0.25) (layer F.Cu) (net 8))
 (segment (start 53.2975 69.9513) (end 53.2975 73.0975) (width 0.25) (layer F.Cu) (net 8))
 (segment (start 53.2975 73.0975) (end 53.5 73.3) (width 0.25) (layer F.Cu) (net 8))
 (segment (start 56 75.8) (end 57.07763 75.8) (width 0.25) (layer F.Cu) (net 9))
 (segment (start 57.07763 75.8) (end 58.53 75.8) (width 0.25) (layer F.Cu) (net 9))
 (segment (start 55.2975 69.9513) (end 55.2975 70.5101) (width 0.25) (layer F.Cu) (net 9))
 (segment (start 55.2975 70.5101) (end 54.75 71.0576) (width 0.25) (layer F.Cu) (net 9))
 (segment (start 54.75 71.0576) (end 54.75 74.55) (width 0.25) (layer F.Cu) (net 9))
 (segment (start 54.75 74.55) (end 55.238001 75.038001) (width 0.25) (layer F.Cu) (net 9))
 (segment (start 55.238001 75.038001) (end 56 75.8) (width 0.25) (layer F.Cu) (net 9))
 (segment (start 57.4563 69.9513) (end 57.4563 72.1863) (width 0.25) (layer F.Cu) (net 10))
 (segment (start 57.4563 72.1863) (end 58.53 73.26) (width 0.25) (layer F.Cu) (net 10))
 (segment (start 56 73.3) (end 58.49 73.3) (width 0.25) (layer F.Cu) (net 10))
 (segment (start 58.49 73.3) (end 58.53 73.26) (width 0.25) (layer F.Cu) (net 10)))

